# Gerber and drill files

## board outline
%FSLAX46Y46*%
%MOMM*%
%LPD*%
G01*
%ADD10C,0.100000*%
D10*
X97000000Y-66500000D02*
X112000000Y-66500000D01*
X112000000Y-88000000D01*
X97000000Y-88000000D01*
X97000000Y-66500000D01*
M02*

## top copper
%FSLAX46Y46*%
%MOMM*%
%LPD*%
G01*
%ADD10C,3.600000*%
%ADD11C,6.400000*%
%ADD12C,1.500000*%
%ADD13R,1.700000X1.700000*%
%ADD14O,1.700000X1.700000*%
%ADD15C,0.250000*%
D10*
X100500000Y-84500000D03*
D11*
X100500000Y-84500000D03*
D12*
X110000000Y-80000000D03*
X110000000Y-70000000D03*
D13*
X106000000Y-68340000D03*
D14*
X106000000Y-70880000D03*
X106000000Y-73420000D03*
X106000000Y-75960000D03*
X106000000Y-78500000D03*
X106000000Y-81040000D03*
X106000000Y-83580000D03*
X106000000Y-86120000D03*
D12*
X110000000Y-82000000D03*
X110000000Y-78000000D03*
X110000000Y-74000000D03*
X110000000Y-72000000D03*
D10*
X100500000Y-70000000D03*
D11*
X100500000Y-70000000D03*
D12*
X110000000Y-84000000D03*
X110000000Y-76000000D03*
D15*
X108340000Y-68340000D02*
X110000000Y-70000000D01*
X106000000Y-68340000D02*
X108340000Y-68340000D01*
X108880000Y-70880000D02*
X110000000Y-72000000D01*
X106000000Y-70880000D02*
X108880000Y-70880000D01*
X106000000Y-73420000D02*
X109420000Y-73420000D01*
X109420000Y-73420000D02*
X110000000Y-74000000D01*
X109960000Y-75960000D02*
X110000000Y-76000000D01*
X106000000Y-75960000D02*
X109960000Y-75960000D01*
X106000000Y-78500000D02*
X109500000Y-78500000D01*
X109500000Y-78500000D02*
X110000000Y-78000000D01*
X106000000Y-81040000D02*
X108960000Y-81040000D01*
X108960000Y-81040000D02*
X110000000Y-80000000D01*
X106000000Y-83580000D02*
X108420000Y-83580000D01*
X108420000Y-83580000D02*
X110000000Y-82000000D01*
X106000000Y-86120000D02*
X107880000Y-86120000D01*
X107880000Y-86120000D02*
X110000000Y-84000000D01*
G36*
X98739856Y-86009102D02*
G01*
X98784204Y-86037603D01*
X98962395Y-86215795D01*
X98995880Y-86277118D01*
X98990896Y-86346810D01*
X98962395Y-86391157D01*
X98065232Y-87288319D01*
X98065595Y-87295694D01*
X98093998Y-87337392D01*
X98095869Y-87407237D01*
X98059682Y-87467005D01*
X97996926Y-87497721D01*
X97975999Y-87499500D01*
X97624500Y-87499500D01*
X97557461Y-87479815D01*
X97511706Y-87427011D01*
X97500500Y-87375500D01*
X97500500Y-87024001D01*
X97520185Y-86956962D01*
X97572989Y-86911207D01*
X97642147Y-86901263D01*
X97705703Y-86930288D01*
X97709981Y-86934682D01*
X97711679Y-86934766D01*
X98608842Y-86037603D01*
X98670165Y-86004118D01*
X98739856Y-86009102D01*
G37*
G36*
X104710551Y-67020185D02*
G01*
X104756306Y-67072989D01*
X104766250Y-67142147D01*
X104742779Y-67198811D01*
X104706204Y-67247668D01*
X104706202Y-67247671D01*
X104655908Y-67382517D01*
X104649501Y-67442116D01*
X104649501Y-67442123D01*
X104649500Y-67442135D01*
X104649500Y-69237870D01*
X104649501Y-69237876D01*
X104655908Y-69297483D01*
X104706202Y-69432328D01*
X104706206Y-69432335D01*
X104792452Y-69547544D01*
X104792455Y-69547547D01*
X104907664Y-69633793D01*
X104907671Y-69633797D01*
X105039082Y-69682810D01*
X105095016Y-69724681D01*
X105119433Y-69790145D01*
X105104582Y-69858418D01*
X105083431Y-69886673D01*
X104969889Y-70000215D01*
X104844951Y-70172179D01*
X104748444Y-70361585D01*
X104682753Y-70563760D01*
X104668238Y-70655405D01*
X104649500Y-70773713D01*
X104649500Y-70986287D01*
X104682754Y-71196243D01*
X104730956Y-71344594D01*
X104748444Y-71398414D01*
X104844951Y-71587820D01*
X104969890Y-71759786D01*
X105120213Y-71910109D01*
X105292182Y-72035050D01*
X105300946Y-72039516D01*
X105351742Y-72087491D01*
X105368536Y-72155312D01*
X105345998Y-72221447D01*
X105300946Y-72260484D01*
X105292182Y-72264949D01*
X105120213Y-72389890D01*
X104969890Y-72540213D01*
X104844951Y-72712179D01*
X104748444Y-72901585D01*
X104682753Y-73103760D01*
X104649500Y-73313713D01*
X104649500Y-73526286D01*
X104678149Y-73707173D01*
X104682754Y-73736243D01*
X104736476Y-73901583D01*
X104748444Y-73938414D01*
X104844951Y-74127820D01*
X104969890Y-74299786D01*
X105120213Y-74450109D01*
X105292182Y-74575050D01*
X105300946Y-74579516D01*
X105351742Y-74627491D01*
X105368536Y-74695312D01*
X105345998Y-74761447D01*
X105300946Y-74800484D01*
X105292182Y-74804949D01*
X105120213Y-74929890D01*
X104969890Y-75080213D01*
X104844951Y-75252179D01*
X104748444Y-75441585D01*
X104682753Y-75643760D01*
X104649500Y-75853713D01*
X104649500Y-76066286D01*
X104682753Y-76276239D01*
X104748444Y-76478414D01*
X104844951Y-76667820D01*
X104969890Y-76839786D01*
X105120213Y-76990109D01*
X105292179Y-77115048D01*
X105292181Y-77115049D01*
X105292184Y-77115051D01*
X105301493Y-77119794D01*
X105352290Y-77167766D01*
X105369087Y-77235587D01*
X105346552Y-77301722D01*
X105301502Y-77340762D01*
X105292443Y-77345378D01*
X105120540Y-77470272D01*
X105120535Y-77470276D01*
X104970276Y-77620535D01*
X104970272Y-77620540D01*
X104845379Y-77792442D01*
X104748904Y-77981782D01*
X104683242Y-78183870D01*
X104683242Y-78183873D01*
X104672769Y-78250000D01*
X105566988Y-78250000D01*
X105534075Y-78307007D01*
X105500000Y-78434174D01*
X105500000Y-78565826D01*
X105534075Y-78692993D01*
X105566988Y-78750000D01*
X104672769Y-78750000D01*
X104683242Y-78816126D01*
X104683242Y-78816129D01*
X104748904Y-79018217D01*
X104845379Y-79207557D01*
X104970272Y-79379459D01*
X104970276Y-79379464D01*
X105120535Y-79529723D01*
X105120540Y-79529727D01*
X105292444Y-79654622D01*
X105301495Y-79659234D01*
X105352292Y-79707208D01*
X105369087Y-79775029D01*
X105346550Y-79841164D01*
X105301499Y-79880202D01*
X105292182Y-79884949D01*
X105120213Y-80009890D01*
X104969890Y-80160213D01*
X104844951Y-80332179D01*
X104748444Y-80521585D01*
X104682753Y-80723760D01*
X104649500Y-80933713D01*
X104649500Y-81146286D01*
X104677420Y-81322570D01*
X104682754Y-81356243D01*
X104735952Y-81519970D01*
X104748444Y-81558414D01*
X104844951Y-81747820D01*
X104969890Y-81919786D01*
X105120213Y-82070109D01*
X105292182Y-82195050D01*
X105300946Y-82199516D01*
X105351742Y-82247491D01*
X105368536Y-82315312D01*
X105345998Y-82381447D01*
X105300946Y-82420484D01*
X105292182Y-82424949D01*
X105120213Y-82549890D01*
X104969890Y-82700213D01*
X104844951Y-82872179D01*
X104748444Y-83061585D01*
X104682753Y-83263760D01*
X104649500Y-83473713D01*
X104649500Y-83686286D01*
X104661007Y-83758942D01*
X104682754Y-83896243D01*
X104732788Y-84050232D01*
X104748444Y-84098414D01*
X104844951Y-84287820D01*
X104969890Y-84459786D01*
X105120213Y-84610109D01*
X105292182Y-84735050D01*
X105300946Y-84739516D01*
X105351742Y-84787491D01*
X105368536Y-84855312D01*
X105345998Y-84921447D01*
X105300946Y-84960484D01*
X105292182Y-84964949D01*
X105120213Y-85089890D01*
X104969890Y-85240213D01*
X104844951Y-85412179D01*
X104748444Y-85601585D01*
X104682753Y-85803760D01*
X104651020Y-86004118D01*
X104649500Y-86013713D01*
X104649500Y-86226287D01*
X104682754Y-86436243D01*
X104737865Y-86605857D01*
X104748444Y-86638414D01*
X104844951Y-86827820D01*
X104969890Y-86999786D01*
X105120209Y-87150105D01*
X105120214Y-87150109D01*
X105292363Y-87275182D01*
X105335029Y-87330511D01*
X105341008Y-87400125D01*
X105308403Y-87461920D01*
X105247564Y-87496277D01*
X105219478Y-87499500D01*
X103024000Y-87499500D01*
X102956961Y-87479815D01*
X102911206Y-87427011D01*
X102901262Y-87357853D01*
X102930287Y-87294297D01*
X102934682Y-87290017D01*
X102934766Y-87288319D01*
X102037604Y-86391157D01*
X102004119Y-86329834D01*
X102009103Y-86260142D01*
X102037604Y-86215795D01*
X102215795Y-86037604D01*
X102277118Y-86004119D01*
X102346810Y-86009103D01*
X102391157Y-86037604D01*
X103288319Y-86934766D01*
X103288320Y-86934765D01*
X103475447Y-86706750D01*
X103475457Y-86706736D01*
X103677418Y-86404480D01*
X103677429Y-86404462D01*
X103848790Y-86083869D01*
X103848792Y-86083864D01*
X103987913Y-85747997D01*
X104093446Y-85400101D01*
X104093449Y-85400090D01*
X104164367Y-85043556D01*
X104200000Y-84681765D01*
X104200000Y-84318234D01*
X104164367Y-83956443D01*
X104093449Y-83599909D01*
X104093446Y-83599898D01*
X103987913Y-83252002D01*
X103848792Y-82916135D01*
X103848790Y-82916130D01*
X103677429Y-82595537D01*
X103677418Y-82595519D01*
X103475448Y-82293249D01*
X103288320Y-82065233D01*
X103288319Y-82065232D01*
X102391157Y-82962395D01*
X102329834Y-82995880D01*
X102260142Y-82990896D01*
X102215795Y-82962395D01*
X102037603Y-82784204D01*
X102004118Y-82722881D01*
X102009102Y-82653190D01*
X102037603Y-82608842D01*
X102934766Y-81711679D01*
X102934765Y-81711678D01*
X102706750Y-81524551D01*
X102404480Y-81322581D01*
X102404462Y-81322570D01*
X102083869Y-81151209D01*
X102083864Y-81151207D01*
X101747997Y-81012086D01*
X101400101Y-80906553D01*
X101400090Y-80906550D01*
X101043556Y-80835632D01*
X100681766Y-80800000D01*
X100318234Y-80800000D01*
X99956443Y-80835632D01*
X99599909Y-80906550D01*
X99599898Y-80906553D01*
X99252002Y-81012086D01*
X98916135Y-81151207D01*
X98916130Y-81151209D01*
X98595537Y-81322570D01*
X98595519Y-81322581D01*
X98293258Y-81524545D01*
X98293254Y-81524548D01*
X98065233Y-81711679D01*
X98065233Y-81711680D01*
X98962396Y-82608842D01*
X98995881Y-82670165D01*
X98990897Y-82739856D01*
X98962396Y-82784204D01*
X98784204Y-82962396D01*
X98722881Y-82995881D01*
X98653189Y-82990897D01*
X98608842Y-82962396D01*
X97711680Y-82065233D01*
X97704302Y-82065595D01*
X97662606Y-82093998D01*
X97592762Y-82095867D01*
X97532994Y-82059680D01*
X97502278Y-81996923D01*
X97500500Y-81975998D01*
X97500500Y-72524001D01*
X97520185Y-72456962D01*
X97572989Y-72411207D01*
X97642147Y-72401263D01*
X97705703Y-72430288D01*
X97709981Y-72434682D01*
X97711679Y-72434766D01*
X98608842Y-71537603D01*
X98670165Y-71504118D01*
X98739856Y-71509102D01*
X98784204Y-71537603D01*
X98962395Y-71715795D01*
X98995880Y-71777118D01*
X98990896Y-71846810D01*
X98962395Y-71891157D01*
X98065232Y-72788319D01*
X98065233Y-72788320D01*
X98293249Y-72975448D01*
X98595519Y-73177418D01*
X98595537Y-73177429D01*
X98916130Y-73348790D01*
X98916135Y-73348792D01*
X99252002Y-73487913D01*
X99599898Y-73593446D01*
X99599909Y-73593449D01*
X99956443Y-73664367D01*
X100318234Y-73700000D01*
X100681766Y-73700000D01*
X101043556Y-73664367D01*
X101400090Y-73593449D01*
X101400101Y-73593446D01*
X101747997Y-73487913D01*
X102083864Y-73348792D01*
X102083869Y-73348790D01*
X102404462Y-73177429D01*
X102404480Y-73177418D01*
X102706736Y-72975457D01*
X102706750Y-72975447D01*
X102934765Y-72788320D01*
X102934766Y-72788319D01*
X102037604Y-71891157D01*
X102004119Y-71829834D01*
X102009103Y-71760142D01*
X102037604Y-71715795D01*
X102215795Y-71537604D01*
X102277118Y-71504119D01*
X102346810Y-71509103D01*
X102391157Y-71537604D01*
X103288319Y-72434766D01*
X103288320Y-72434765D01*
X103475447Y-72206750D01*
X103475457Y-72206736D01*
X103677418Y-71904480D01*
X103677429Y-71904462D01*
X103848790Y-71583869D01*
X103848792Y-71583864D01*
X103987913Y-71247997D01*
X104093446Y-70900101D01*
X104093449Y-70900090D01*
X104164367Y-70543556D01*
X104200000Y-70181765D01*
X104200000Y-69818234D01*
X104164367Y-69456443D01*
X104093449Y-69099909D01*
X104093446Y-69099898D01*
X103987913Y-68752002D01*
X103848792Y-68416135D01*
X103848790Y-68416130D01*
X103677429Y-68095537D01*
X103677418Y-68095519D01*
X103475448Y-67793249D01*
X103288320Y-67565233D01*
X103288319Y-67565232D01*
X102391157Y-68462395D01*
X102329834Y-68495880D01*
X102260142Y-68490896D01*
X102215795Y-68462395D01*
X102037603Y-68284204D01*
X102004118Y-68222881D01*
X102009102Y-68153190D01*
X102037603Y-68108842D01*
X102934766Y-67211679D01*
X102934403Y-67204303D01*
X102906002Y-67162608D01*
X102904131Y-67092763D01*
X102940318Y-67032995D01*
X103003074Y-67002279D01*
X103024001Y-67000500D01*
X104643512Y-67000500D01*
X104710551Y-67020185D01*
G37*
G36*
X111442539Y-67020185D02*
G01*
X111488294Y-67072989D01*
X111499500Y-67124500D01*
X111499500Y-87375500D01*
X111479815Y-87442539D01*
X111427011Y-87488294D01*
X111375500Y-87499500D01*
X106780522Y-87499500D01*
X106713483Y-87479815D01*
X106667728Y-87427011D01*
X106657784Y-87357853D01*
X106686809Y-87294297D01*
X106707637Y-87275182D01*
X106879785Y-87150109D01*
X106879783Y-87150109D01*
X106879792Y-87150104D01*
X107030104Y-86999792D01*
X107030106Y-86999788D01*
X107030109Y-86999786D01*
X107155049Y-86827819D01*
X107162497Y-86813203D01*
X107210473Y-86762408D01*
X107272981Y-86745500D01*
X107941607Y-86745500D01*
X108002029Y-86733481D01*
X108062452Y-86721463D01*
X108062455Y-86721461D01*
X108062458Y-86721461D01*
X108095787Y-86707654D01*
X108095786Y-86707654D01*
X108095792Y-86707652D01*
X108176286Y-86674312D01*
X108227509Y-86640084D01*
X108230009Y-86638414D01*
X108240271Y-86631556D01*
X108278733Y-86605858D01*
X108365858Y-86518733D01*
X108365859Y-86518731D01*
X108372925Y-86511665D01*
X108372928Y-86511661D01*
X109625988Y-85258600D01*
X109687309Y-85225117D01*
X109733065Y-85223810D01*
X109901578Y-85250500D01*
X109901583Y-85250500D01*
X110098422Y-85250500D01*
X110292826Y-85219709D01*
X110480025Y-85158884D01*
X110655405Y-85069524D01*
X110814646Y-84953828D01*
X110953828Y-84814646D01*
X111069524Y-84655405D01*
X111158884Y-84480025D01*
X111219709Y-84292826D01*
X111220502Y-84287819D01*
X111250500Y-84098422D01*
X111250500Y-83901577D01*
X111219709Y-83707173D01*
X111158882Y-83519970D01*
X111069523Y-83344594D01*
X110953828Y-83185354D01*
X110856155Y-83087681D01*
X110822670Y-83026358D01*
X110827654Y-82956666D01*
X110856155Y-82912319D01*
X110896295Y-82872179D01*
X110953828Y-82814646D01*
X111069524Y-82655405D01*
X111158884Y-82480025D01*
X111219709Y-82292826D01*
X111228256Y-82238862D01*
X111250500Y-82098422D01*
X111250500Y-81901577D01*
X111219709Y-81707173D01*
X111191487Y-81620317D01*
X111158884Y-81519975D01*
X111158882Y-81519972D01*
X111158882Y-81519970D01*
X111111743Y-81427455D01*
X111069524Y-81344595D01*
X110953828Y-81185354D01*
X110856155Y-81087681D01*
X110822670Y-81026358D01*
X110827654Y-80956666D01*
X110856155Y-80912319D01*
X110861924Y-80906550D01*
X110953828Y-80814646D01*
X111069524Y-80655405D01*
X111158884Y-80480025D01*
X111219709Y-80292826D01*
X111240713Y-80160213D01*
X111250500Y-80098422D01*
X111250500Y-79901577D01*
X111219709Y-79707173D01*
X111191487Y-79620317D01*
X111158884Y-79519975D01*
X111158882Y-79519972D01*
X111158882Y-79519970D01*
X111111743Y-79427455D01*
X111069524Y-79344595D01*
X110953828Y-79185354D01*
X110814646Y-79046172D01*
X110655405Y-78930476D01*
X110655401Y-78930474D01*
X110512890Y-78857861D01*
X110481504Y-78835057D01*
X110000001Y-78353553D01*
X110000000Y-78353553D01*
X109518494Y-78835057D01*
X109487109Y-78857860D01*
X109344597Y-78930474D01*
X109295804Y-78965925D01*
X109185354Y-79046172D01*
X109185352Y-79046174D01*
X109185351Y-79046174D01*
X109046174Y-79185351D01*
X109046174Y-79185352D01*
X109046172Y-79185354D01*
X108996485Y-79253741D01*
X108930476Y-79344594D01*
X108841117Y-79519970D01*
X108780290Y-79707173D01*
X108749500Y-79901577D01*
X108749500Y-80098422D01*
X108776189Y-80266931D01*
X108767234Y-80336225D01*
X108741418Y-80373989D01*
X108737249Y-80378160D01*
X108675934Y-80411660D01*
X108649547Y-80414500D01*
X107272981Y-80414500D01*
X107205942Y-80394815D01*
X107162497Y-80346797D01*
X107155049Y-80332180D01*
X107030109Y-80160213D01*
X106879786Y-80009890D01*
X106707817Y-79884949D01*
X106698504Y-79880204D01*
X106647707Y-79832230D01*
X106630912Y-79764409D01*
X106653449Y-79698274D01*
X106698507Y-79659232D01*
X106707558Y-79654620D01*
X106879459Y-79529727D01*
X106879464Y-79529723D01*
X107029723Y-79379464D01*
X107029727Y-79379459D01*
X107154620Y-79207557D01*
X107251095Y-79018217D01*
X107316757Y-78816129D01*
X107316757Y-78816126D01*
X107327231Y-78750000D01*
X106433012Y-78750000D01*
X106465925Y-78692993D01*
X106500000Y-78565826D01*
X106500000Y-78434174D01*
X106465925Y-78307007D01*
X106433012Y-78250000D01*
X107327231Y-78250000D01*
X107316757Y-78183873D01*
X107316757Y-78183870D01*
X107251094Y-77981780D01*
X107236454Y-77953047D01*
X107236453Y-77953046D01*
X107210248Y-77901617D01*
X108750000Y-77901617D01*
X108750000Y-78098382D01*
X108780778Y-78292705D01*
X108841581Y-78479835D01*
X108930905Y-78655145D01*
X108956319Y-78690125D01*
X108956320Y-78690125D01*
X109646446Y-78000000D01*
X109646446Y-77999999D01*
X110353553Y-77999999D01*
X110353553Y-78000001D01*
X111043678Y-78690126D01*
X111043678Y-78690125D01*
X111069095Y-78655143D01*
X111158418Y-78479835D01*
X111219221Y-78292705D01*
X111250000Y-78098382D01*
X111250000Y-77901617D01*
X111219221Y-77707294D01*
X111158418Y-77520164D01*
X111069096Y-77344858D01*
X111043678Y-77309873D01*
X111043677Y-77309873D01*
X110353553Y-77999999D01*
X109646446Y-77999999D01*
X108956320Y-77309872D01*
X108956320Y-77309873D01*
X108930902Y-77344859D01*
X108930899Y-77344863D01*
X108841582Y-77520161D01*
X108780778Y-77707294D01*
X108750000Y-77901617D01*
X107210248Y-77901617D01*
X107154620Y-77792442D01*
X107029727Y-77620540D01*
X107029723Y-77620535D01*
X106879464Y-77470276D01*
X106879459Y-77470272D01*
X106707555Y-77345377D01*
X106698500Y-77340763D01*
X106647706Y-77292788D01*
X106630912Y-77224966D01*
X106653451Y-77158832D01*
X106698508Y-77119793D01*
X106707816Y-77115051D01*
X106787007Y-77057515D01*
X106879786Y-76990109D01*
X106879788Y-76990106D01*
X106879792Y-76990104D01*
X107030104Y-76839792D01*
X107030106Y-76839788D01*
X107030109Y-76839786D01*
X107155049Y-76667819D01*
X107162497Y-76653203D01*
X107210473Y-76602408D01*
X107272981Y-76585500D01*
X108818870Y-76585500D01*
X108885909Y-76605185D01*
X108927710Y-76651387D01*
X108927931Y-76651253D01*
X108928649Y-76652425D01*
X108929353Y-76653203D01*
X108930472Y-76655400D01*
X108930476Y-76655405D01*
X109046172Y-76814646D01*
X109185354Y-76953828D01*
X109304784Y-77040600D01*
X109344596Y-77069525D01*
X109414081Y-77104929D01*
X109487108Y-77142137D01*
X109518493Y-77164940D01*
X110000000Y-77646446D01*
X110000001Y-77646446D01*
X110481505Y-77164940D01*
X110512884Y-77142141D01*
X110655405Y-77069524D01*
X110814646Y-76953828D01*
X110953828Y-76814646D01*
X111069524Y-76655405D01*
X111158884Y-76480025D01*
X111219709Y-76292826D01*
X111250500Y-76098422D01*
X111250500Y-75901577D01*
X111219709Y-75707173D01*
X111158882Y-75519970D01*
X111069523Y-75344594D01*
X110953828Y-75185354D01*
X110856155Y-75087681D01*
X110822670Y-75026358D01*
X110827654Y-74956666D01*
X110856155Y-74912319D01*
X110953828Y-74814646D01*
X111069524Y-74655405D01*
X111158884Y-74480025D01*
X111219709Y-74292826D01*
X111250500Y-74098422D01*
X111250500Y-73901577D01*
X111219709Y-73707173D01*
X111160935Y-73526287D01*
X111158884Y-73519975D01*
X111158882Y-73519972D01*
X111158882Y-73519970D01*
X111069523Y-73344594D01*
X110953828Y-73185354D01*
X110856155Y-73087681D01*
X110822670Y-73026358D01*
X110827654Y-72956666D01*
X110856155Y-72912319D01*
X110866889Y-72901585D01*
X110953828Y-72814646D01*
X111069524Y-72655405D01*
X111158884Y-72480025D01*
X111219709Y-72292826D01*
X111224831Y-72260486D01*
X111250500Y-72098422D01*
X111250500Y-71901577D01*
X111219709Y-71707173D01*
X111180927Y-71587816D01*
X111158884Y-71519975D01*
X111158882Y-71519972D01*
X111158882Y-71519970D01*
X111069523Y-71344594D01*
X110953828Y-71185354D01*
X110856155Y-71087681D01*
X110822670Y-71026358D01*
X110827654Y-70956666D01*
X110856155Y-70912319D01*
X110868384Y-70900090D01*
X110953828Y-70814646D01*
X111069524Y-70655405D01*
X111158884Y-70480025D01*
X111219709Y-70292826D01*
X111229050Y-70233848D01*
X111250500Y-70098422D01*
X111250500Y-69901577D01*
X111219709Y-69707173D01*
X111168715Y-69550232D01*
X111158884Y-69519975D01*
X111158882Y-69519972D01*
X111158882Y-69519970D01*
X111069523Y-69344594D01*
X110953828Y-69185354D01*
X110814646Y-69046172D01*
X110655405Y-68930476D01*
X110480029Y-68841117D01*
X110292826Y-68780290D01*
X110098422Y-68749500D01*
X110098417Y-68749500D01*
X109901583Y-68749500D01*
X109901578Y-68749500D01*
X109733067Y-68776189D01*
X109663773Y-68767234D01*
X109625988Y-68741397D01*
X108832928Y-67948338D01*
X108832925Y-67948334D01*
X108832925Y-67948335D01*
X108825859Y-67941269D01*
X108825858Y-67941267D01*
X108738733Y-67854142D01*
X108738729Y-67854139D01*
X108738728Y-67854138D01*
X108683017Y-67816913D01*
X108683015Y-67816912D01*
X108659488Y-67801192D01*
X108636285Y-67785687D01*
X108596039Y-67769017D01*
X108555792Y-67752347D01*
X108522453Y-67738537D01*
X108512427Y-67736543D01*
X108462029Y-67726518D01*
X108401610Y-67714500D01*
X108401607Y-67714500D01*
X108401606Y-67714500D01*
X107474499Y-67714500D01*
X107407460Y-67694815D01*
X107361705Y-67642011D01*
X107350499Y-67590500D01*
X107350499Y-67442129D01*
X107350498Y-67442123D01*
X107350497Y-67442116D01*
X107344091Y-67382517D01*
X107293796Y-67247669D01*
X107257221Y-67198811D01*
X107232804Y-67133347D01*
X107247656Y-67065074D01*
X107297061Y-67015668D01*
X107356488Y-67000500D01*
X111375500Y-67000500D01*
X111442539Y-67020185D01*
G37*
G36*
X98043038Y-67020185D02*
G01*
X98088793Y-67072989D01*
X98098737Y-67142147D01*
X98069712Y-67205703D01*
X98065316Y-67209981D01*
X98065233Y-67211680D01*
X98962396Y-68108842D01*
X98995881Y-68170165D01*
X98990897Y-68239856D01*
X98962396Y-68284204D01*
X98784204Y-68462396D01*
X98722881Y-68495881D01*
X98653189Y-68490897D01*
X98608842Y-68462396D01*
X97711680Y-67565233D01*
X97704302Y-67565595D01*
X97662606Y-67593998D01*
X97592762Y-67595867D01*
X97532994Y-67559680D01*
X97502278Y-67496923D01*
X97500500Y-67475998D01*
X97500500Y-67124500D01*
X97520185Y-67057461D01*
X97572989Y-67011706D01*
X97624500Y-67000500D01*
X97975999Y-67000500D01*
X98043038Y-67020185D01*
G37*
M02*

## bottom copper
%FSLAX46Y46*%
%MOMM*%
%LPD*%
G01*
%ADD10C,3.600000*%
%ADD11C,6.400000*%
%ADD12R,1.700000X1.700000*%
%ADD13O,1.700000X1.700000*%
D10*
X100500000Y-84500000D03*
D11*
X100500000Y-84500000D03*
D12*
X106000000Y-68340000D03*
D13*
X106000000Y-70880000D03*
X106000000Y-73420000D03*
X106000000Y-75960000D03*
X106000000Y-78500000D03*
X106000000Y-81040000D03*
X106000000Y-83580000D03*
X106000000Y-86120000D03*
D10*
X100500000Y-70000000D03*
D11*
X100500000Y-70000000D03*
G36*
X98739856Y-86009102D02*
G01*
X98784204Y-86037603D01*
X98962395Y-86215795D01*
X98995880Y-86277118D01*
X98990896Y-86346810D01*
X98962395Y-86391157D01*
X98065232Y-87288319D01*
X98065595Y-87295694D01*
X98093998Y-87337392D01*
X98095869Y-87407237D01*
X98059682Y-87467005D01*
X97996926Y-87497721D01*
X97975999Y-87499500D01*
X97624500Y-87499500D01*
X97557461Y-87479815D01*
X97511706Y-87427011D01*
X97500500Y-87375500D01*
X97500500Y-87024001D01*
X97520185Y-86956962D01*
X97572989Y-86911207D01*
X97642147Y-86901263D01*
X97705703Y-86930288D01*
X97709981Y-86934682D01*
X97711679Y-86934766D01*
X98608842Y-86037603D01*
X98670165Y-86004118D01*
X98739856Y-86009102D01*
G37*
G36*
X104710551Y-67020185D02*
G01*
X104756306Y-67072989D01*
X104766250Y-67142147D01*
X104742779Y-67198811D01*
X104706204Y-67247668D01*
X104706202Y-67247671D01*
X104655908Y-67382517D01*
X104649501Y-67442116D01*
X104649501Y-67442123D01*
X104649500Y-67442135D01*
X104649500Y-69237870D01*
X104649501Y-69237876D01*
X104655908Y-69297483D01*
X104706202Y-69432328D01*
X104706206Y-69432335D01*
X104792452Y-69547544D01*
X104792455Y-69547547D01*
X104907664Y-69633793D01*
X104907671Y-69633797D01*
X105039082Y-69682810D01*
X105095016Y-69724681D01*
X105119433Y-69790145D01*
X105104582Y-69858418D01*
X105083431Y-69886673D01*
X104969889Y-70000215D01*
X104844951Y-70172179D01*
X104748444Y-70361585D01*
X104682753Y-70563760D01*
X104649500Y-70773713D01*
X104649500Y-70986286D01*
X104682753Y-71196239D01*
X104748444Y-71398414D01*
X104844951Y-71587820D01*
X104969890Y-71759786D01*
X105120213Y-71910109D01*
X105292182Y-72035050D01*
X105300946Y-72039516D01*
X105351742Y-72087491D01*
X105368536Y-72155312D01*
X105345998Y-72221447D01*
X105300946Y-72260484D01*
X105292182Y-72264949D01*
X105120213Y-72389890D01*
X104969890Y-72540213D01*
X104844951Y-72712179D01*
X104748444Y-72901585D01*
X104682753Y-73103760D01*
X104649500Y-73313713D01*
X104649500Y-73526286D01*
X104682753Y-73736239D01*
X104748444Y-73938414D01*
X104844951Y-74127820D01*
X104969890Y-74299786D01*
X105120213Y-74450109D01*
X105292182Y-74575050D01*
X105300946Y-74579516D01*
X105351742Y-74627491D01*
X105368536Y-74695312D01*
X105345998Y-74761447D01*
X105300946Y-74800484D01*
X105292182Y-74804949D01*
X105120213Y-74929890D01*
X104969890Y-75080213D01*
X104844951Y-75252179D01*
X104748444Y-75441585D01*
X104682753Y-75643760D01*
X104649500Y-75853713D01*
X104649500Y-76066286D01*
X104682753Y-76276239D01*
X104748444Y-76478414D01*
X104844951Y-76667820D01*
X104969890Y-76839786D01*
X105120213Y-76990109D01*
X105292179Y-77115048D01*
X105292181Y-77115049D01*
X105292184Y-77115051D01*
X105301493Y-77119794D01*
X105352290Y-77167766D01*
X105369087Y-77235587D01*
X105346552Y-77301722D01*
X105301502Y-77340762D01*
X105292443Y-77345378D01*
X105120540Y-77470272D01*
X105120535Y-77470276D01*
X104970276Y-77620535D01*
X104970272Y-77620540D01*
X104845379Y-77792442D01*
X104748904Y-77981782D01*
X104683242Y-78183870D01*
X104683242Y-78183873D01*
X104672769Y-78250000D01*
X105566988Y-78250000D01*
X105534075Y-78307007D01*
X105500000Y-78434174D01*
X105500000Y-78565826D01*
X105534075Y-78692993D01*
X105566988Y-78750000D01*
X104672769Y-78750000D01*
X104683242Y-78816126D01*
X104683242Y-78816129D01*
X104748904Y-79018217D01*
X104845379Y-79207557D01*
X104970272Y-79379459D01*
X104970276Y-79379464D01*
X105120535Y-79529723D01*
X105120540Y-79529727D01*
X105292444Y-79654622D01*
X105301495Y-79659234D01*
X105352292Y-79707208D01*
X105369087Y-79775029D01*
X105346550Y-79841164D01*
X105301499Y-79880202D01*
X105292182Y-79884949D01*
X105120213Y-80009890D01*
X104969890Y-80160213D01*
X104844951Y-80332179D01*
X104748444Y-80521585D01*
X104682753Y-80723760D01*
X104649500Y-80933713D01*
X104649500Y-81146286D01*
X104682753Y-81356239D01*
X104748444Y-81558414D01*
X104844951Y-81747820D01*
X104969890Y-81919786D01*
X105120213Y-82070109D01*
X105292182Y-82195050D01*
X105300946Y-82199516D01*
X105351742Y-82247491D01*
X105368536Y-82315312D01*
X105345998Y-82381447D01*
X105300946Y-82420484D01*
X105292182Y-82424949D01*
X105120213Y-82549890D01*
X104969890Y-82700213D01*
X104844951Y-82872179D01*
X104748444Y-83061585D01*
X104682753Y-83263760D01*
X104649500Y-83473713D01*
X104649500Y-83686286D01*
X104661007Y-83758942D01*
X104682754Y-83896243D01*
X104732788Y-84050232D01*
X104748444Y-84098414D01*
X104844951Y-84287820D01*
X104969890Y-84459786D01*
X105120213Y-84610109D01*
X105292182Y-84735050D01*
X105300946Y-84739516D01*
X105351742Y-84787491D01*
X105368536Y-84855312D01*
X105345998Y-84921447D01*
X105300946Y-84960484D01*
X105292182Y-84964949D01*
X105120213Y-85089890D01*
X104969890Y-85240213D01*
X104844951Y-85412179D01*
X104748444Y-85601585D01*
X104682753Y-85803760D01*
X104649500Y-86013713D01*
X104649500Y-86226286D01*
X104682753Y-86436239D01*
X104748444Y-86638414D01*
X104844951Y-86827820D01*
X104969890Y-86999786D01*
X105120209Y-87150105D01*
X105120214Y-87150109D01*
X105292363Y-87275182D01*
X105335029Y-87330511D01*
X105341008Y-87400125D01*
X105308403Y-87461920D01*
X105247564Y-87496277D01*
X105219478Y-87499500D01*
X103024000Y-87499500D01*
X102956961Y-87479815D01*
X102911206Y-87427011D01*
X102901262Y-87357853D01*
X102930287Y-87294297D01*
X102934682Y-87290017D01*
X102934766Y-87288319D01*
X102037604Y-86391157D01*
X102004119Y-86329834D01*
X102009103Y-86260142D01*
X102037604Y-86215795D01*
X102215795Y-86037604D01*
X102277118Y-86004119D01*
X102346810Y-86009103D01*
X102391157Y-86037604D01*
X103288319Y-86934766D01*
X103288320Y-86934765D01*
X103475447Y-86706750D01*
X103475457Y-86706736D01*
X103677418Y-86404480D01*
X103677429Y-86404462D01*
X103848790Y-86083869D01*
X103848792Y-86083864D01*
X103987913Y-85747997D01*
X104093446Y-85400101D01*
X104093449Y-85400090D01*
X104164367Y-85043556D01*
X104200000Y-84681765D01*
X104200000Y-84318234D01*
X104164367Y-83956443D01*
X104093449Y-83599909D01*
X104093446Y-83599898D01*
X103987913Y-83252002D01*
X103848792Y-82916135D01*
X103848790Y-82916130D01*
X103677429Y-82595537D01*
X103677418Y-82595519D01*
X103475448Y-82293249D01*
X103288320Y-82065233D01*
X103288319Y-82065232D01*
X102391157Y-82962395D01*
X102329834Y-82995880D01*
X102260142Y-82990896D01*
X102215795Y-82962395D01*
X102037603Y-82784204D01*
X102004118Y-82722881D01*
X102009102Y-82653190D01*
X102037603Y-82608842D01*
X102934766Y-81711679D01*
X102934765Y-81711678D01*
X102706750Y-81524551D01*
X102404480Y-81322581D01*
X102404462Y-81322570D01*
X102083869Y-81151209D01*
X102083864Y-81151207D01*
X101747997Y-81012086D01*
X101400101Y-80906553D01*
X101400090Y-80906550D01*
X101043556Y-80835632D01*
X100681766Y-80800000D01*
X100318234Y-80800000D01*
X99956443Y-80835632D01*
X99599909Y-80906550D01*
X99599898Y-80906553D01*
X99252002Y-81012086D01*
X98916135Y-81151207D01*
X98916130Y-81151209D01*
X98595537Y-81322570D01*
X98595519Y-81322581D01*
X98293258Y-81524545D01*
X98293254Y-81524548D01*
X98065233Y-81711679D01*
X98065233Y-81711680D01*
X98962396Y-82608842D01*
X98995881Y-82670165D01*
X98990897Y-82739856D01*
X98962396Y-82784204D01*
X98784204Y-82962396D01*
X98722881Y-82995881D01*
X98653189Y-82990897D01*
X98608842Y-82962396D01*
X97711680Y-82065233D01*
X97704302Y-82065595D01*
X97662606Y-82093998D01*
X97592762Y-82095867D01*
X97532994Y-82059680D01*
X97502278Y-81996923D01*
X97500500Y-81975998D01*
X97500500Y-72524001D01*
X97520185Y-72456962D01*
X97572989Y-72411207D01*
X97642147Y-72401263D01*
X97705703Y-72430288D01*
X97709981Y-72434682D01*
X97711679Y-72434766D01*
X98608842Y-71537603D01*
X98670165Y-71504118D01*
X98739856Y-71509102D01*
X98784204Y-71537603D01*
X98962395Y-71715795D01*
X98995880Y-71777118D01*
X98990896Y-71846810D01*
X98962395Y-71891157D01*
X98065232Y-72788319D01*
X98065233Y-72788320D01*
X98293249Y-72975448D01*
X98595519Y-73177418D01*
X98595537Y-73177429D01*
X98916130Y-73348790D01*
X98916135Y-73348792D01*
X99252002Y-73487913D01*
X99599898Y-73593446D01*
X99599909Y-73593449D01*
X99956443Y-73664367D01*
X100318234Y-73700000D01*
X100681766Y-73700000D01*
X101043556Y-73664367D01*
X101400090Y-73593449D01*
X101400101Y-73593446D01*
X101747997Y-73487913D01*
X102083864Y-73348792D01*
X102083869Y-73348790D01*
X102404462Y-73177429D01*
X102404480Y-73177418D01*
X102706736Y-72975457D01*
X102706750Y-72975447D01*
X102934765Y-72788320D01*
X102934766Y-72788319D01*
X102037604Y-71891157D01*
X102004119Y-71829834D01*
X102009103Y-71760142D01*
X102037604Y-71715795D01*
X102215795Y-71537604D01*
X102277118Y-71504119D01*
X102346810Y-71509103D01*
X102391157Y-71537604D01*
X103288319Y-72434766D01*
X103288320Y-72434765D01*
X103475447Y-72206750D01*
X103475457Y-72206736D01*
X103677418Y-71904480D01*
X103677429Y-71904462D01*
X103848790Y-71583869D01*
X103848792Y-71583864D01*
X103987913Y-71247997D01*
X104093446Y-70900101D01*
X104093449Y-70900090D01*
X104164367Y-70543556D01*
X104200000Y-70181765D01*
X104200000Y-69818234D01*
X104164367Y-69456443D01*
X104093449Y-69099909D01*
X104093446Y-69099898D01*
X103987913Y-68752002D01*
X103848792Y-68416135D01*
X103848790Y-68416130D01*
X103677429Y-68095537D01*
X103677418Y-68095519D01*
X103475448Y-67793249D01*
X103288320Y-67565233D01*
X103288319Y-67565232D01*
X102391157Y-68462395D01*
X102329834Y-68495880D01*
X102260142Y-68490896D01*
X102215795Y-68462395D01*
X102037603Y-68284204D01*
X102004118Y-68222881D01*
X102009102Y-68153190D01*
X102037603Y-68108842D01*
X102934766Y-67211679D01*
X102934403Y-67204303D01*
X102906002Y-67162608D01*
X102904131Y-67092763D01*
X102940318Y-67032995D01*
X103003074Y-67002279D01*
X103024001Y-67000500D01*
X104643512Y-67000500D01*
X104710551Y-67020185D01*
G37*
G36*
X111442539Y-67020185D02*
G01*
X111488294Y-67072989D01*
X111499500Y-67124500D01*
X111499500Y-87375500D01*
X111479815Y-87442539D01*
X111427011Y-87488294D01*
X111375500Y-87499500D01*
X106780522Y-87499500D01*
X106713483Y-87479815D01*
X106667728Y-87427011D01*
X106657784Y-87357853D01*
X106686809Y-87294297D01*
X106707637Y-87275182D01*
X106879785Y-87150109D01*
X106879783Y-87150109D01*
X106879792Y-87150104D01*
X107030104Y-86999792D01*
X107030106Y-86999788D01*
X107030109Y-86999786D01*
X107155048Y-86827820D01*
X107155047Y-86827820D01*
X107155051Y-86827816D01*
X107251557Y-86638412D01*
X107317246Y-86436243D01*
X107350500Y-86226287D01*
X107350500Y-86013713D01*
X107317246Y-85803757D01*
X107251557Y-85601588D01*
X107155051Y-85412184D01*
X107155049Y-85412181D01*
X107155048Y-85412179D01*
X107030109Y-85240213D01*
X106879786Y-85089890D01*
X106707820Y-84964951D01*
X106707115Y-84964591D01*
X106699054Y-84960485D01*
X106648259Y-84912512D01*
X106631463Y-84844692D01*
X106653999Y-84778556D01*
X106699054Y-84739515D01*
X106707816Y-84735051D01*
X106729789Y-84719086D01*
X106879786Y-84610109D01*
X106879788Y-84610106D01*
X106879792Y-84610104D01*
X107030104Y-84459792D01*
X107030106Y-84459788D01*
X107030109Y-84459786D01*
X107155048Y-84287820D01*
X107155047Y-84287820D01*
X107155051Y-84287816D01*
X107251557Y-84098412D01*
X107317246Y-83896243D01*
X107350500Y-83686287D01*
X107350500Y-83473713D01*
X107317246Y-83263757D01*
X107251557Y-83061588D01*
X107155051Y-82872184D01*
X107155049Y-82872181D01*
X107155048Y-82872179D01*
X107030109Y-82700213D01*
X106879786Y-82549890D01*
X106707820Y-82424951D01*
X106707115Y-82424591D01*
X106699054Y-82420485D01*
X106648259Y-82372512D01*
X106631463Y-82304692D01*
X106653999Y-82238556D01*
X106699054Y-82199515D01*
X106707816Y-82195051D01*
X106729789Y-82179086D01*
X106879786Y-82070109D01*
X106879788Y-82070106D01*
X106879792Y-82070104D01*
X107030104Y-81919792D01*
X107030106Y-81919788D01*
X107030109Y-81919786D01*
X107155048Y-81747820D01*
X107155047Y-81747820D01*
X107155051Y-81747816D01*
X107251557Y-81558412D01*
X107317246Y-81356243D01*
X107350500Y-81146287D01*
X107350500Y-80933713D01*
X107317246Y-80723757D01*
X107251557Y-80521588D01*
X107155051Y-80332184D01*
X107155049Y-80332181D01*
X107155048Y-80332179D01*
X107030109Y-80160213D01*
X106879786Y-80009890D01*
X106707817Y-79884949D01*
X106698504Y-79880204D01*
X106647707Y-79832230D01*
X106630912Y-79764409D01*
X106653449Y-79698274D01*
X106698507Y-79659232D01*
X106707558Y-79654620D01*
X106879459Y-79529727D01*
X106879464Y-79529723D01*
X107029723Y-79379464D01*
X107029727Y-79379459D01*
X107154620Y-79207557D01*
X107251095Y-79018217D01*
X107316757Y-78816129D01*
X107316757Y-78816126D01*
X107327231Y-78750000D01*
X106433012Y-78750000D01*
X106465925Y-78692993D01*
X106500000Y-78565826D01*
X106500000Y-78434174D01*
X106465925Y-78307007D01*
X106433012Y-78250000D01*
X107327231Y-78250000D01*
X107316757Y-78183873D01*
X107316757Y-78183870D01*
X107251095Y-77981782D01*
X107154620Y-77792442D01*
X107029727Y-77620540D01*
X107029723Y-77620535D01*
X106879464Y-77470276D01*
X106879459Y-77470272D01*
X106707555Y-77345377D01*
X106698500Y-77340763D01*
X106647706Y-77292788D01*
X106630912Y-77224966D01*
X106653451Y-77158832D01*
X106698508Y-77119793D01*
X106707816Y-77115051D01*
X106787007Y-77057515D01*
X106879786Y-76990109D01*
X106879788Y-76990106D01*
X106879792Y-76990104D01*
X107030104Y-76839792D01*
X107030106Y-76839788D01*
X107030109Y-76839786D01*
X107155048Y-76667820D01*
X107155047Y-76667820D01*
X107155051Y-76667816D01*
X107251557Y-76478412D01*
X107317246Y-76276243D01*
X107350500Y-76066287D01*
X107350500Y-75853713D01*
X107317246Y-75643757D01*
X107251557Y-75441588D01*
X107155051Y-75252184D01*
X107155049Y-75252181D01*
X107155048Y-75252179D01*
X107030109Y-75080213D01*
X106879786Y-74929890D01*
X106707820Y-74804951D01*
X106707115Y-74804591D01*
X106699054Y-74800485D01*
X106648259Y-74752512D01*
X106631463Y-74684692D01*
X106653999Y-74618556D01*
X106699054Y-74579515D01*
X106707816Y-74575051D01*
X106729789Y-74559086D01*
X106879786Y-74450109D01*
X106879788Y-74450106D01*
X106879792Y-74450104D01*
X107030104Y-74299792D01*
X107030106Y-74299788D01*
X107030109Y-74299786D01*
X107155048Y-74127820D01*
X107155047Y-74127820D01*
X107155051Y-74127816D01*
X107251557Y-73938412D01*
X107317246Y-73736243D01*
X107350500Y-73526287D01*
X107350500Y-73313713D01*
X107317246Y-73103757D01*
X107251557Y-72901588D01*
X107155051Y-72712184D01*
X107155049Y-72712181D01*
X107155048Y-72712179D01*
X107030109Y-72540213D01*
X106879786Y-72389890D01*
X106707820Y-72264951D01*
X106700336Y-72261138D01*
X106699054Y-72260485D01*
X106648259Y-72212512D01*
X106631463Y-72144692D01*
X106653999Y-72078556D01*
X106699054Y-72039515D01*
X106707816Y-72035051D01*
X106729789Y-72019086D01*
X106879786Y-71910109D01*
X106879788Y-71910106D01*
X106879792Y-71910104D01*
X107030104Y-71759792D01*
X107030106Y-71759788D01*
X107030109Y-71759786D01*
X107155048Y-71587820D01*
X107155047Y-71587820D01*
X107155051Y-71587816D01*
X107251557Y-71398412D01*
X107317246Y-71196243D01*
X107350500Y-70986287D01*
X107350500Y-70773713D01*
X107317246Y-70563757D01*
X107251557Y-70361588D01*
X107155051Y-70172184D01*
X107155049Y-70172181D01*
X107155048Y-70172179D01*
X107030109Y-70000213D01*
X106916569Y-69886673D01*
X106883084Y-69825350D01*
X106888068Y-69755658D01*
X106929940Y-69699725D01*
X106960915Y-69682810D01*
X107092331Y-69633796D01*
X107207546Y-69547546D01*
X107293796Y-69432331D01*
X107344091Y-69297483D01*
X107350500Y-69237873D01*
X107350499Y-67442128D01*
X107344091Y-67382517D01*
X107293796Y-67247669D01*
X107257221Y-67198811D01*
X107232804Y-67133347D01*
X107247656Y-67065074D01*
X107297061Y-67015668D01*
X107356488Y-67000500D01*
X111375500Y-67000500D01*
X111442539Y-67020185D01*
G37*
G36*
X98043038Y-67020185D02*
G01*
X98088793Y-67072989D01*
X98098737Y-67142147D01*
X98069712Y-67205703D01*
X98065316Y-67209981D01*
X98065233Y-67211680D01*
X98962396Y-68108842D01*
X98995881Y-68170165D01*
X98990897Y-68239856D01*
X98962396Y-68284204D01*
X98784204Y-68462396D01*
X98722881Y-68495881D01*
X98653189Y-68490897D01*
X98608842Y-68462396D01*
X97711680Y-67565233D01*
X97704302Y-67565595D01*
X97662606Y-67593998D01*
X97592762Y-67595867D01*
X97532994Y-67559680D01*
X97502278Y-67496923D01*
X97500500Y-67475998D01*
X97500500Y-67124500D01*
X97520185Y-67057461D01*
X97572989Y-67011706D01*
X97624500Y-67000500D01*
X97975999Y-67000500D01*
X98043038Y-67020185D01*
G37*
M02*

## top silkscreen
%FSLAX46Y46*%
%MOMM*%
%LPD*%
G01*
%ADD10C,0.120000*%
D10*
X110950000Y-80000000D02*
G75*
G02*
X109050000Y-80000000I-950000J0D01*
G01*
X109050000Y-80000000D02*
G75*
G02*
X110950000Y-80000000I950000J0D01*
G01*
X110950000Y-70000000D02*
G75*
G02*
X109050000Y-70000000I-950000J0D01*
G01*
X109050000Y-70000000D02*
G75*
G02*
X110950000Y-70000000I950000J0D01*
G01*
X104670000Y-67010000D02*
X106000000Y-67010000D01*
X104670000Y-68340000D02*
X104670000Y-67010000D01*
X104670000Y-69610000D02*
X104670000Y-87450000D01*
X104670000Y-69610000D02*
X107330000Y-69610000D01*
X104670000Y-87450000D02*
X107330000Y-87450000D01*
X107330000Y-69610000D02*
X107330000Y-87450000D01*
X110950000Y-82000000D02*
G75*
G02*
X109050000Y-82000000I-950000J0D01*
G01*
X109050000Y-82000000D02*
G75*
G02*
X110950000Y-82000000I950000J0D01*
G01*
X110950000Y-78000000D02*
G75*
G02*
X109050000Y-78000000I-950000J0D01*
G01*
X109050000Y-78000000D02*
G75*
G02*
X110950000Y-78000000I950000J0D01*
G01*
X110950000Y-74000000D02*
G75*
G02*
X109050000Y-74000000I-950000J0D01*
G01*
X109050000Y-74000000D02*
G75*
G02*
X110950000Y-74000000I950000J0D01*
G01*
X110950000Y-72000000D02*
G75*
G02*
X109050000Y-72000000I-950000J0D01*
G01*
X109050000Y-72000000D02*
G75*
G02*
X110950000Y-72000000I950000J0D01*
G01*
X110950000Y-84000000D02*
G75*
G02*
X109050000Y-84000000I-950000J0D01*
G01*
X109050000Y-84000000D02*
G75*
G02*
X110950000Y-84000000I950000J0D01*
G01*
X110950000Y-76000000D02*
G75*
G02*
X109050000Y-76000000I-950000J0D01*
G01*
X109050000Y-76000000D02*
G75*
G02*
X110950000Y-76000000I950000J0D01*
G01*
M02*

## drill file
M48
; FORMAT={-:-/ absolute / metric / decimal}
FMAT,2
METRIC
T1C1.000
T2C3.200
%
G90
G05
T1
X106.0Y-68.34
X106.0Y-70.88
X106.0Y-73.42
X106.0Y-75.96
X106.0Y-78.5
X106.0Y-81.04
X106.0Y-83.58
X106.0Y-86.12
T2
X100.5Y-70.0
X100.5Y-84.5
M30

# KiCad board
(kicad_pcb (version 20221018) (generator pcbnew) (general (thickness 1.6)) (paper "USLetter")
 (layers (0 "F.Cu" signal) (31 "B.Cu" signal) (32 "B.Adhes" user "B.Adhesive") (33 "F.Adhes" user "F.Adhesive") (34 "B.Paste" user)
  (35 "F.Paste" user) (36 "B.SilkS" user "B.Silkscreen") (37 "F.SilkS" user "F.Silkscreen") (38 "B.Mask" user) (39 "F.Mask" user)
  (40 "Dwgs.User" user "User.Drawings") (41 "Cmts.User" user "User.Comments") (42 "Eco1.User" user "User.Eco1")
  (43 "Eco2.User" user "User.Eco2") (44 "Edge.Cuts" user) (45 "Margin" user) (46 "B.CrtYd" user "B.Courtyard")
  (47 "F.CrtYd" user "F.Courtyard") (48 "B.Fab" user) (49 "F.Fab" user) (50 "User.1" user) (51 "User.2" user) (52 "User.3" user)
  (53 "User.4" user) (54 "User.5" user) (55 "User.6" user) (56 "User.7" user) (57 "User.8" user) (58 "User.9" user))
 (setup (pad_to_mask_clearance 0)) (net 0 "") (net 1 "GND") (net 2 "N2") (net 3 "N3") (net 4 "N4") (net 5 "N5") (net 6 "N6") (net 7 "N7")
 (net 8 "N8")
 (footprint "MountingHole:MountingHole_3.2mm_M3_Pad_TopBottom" (layer "F.Cu") (at 100.5 84.5)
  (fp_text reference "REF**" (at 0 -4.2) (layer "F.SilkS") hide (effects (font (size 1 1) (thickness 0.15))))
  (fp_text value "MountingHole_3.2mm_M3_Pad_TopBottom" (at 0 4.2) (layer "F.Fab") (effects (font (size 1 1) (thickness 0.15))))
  (pad "1" thru_hole circle (at 0 0) (size 3.6 3.6) (drill 3.2) (layers "*.Cu" "*.Mask"))
  (pad "1" connect circle (at 0 0) (size 6.4 6.4) (layers "F.Cu" "F.Mask") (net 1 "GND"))
  (pad "1" connect circle (at 0 0) (size 6.4 6.4) (layers "B.Cu" "B.Mask") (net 1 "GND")))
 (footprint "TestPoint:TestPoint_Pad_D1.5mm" (layer "F.Cu") (at 110 80)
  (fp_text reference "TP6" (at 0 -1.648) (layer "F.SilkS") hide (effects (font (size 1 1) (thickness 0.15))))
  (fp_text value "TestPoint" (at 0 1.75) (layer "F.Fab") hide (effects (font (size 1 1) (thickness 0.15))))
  (fp_circle (center 0 0) (end 0 0.95) (stroke (width 0.12) (type solid)) (fill none) (layer "F.SilkS"))
  (pad "1" smd circle (at 0 0) (size 1.5 1.5) (layers "F.Cu" "F.Mask") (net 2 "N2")))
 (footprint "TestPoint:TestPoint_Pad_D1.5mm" (layer "F.Cu") (at 110 70)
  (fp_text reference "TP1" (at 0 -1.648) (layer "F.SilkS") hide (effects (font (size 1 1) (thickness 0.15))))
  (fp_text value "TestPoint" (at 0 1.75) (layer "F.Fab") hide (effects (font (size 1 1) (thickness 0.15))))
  (fp_circle (center 0 0) (end 0 0.95) (stroke (width 0.12) (type solid)) (fill none) (layer "F.SilkS"))
  (pad "1" smd circle (at 0 0) (size 1.5 1.5) (layers "F.Cu" "F.Mask") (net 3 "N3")))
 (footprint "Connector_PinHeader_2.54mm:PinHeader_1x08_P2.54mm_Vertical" (layer "F.Cu") (at 106 68.34)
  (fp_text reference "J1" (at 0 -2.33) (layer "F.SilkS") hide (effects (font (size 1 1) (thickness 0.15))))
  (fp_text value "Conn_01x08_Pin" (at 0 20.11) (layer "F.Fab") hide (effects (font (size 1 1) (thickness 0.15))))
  (fp_line (start -1.33 -1.33) (end 0 -1.33) (stroke (width 0.12) (type solid)) (layer "F.SilkS"))
  (fp_line (start -1.33 0) (end -1.33 -1.33) (stroke (width 0.12) (type solid)) (layer "F.SilkS"))
  (fp_line (start -1.33 1.27) (end -1.33 19.11) (stroke (width 0.12) (type solid)) (layer "F.SilkS"))
  (fp_line (start -1.33 1.27) (end 1.33 1.27) (stroke (width 0.12) (type solid)) (layer "F.SilkS"))
  (fp_line (start -1.33 19.11) (end 1.33 19.11) (stroke (width 0.12) (type solid)) (layer "F.SilkS"))
  (fp_line (start 1.33 1.27) (end 1.33 19.11) (stroke (width 0.12) (type solid)) (layer "F.SilkS"))
  (pad "1" thru_hole rect (at 0 0) (size 1.7 1.7) (drill 1) (layers "*.Cu" "*.Mask") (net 3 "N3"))
  (pad "2" thru_hole oval (at 0 2.54) (size 1.7 1.7) (drill 1) (layers "*.Cu" "*.Mask") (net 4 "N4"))
  (pad "3" thru_hole oval (at 0 5.08) (size 1.7 1.7) (drill 1) (layers "*.Cu" "*.Mask") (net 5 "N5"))
  (pad "4" thru_hole oval (at 0 7.62) (size 1.7 1.7) (drill 1) (layers "*.Cu" "*.Mask") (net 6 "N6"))
  (pad "5" thru_hole oval (at 0 10.16) (size 1.7 1.7) (drill 1) (layers "*.Cu" "*.Mask") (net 1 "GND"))
  (pad "6" thru_hole oval (at 0 12.7) (size 1.7 1.7) (drill 1) (layers "*.Cu" "*.Mask") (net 2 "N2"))
  (pad "7" thru_hole oval (at 0 15.24) (size 1.7 1.7) (drill 1) (layers "*.Cu" "*.Mask") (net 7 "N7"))
  (pad "8" thru_hole oval (at 0 17.78) (size 1.7 1.7) (drill 1) (layers "*.Cu" "*.Mask") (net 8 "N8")))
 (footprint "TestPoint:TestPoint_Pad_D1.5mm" (layer "F.Cu") (at 110 82)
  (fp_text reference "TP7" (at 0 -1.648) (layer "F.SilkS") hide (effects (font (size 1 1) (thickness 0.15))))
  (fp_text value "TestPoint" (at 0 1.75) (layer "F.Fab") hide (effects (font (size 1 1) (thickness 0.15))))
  (fp_circle (center 0 0) (end 0 0.95) (stroke (width 0.12) (type solid)) (fill none) (layer "F.SilkS"))
  (pad "1" smd circle (at 0 0) (size 1.5 1.5) (layers "F.Cu" "F.Mask") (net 7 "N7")))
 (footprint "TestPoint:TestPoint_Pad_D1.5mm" (layer "F.Cu") (at 110 78)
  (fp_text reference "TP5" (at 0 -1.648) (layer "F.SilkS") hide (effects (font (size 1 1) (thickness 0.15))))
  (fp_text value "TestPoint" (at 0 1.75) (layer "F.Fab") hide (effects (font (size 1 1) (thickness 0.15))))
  (fp_circle (center 0 0) (end 0 0.95) (stroke (width 0.12) (type solid)) (fill none) (layer "F.SilkS"))
  (pad "1" smd circle (at 0 0) (size 1.5 1.5) (layers "F.Cu" "F.Mask") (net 1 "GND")))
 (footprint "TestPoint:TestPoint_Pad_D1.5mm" (layer "F.Cu") (at 110 74)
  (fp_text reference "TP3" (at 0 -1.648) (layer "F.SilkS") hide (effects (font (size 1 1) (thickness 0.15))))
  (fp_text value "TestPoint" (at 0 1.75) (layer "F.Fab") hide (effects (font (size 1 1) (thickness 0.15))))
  (fp_circle (center 0 0) (end 0 0.95) (stroke (width 0.12) (type solid)) (fill none) (layer "F.SilkS"))
  (pad "1" smd circle (at 0 0) (size 1.5 1.5) (layers "F.Cu" "F.Mask") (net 5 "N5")))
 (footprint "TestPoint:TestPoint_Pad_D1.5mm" (layer "F.Cu") (at 110 72)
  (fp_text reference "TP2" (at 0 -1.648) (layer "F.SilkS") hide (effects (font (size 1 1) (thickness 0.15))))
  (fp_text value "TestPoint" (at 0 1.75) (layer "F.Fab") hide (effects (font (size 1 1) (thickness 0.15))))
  (fp_circle (center 0 0) (end 0 0.95) (stroke (width 0.12) (type solid)) (fill none) (layer "F.SilkS"))
  (pad "1" smd circle (at 0 0) (size 1.5 1.5) (layers "F.Cu" "F.Mask") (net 4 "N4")))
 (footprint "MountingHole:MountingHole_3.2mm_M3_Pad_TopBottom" (layer "F.Cu") (at 100.5 70)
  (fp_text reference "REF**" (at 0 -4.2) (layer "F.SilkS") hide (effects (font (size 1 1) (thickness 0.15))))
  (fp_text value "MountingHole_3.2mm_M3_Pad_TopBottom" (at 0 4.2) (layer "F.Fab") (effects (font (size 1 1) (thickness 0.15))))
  (pad "1" thru_hole circle (at 0 0) (size 3.6 3.6) (drill 3.2) (layers "*.Cu" "*.Mask"))
  (pad "1" connect circle (at 0 0) (size 6.4 6.4) (layers "F.Cu" "F.Mask") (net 1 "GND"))
  (pad "1" connect circle (at 0 0) (size 6.4 6.4) (layers "B.Cu" "B.Mask") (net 1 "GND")))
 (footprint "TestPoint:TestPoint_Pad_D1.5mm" (layer "F.Cu") (at 110 84)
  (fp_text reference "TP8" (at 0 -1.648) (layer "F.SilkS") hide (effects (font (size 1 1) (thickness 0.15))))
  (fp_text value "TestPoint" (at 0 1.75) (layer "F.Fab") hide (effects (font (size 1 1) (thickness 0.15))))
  (fp_circle (center 0 0) (end 0 0.95) (stroke (width 0.12) (type solid)) (fill none) (layer "F.SilkS"))
  (pad "1" smd circle (at 0 0) (size 1.5 1.5) (layers "F.Cu" "F.Mask") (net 8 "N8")))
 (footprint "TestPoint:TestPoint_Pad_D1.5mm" (layer "F.Cu") (at 110 76)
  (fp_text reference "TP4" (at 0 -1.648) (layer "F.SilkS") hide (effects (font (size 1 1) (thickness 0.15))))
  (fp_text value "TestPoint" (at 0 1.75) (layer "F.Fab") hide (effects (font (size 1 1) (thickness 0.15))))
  (fp_circle (center 0 0) (end 0 0.95) (stroke (width 0.12) (type solid)) (fill none) (layer "F.SilkS"))
  (pad "1" smd circle (at 0 0) (size 1.5 1.5) (layers "F.Cu" "F.Mask") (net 6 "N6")))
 (gr_rect (start 97 66.5) (end 112 88) (stroke (width 0.1) (type default)) (fill none) (layer "Edge.Cuts"))
 (segment (start 108.34 68.34) (end 110 70) (width 0.25) (layer "F.Cu") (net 3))
 (segment (start 106 68.34) (end 108.34 68.34) (width 0.25) (layer "F.Cu") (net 3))
 (segment (start 108.88 70.88) (end 110 72) (width 0.25) (layer "F.Cu") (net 4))
 (segment (start 106 70.88) (end 108.88 70.88) (width 0.25) (layer "F.Cu") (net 4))
 (segment (start 106 73.42) (end 109.42 73.42) (width 0.25) (layer "F.Cu") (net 5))
 (segment (start 109.42 73.42) (end 110 74) (width 0.25) (layer "F.Cu") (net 5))
 (segment (start 109.96 75.96) (end 110 76) (width 0.25) (layer "F.Cu") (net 6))
 (segment (start 106 75.96) (end 109.96 75.96) (width 0.25) (layer "F.Cu") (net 6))
 (segment (start 106 78.5) (end 109.5 78.5) (width 0.25) (layer "F.Cu") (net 1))
 (segment (start 109.5 78.5) (end 110 78) (width 0.25) (layer "F.Cu") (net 1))
 (segment (start 106 81.04) (end 108.96 81.04) (width 0.25) (layer "F.Cu") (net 2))
 (segment (start 108.96 81.04) (end 110 80) (width 0.25) (layer "F.Cu") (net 2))
 (segment (start 106 83.58) (end 108.42 83.58) (width 0.25) (layer "F.Cu") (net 7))
 (segment (start 108.42 83.58) (end 110 82) (width 0.25) (layer "F.Cu") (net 7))
 (segment (start 106 86.12) (end 107.88 86.12) (width 0.25) (layer "F.Cu") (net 8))
 (segment (start 107.88 86.12) (end 110 84) (width 0.25) (layer "F.Cu") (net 8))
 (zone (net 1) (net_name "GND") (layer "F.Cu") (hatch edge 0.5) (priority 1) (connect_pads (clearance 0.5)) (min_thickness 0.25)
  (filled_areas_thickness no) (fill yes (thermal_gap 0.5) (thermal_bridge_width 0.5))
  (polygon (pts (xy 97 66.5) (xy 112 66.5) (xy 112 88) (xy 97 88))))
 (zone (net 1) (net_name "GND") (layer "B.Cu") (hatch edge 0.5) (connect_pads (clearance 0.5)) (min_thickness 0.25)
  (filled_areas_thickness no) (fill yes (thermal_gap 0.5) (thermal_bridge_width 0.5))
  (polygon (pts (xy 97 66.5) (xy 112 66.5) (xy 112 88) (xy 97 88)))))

